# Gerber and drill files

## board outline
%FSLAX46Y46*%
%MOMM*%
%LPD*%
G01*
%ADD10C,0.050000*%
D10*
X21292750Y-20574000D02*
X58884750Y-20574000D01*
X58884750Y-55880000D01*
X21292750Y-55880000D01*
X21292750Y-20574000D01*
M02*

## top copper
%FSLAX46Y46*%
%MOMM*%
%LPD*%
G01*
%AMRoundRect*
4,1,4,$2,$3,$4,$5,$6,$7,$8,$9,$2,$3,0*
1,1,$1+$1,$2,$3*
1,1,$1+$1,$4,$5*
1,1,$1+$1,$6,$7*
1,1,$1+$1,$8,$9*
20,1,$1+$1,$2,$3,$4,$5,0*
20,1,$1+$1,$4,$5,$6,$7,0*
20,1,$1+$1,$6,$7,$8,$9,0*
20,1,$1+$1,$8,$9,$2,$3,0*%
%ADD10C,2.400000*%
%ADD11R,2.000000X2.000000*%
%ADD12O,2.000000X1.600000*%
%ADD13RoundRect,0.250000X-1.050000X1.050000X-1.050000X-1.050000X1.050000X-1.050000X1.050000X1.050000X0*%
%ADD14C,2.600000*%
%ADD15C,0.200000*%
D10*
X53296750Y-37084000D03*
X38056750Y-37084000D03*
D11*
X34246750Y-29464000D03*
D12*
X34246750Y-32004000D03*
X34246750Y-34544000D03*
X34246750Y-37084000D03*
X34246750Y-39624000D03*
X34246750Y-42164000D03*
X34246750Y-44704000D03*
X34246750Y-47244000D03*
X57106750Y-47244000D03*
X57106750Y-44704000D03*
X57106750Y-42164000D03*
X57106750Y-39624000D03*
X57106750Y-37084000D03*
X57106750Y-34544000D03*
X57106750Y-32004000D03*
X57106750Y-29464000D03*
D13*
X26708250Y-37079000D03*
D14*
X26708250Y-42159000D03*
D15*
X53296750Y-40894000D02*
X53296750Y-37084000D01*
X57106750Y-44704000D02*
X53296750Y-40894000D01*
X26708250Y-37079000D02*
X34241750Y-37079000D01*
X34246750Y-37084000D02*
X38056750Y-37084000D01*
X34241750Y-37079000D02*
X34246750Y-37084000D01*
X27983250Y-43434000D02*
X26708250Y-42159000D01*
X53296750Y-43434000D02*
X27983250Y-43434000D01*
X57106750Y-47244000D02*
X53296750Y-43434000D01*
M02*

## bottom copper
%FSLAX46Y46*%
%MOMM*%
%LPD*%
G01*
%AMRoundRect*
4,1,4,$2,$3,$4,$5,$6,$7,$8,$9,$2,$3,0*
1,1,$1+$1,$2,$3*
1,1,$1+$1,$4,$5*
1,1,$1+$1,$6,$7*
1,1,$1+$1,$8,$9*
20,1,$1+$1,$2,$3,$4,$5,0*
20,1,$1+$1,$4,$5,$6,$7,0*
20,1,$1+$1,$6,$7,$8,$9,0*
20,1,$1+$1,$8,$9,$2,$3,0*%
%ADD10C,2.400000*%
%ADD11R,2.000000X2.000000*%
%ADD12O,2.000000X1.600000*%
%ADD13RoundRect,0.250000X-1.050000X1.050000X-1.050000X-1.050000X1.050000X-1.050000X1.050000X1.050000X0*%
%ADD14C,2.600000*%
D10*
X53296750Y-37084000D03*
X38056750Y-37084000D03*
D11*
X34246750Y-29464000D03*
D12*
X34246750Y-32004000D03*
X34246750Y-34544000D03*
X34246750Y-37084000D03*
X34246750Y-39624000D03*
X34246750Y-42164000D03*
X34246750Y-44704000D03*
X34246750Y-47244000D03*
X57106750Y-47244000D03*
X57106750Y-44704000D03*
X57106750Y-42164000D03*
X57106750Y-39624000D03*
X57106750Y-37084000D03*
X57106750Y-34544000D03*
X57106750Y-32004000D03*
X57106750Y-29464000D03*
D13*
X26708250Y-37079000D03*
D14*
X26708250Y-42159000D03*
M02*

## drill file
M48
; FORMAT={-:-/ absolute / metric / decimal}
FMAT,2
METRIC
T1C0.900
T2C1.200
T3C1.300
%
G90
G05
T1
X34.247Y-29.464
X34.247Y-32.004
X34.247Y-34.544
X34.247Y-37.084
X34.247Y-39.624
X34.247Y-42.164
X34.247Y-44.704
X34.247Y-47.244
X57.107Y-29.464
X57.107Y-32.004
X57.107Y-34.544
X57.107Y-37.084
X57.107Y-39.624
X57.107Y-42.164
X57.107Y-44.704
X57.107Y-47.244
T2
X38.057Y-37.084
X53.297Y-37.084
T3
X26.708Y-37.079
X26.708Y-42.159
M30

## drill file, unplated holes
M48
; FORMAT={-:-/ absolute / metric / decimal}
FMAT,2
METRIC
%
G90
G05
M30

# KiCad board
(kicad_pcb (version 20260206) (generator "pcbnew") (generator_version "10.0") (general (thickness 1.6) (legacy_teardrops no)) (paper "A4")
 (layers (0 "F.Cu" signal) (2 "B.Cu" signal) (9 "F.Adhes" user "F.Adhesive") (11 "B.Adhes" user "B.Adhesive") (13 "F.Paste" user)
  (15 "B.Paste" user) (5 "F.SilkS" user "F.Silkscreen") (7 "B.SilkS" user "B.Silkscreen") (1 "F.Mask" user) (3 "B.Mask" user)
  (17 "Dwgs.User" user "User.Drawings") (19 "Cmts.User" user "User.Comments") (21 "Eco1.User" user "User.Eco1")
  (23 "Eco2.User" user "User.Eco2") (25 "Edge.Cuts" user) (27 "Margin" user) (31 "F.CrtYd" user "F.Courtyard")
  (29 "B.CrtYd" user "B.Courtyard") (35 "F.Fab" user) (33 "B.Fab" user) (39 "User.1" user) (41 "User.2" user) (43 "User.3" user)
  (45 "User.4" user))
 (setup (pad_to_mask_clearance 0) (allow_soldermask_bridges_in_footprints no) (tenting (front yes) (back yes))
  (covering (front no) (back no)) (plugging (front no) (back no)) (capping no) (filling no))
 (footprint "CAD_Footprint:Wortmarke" (layer "F.Cu") (at 26.924 49.022)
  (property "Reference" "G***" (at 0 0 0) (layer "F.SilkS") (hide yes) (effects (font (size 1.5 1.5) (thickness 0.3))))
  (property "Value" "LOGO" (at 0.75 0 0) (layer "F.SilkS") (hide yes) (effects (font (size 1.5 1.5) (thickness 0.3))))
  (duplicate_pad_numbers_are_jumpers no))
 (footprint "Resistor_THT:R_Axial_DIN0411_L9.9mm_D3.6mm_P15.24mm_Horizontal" (layer "F.Cu") (at 53.29675 37.084 180)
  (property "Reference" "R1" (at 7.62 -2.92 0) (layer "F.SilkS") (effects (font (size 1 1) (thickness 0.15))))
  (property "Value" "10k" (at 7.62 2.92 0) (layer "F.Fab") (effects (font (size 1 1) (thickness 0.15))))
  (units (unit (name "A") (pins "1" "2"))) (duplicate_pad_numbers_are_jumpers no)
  (pad "1" thru_hole circle (at 0 0 180) (size 2.4 2.4) (drill 1.2) (layers "*.Cu" "*.Mask") (remove_unused_layers no) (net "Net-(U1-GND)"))
  (pad "2" thru_hole circle (at 15.24 0 180) (size 2.4 2.4) (drill 1.2) (layers "*.Cu" "*.Mask") (remove_unused_layers no)
   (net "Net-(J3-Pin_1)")))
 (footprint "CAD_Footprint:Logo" (layer "F.Cu") (at 26.924 27.432)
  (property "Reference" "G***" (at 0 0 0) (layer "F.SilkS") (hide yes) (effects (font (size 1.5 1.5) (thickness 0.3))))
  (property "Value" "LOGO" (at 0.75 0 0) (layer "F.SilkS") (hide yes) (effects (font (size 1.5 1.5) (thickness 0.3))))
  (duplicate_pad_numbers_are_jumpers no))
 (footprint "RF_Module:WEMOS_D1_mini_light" (layer "F.Cu") (at 34.24675 29.464)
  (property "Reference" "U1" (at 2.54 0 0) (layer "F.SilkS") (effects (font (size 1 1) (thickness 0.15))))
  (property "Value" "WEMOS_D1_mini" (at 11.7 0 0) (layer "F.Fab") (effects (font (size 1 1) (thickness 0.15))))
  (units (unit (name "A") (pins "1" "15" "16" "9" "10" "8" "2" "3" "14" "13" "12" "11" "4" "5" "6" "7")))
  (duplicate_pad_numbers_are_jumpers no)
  (pad "1" thru_hole rect (at 0 0) (size 2 2) (drill 0.9) (layers "*.Cu" "*.Mask") (remove_unused_layers no)
   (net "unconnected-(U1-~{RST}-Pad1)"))
  (pad "2" thru_hole oval (at 0 2.54) (size 2 1.6) (drill 0.9) (layers "*.Cu" "*.Mask") (remove_unused_layers no)
   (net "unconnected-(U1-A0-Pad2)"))
  (pad "3" thru_hole oval (at 0 5.08) (size 2 1.6) (drill 0.9) (layers "*.Cu" "*.Mask") (remove_unused_layers no)
   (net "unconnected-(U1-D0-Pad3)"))
  (pad "4" thru_hole oval (at 0 7.62) (size 2 1.6) (drill 0.9) (layers "*.Cu" "*.Mask") (remove_unused_layers no) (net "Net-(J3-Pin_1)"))
  (pad "5" thru_hole oval (at 0 10.16) (size 2 1.6) (drill 0.9) (layers "*.Cu" "*.Mask") (remove_unused_layers no)
   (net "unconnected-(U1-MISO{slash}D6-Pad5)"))
  (pad "6" thru_hole oval (at 0 12.7) (size 2 1.6) (drill 0.9) (layers "*.Cu" "*.Mask") (remove_unused_layers no)
   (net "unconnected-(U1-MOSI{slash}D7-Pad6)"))
  (pad "7" thru_hole oval (at 0 15.24) (size 2 1.6) (drill 0.9) (layers "*.Cu" "*.Mask") (remove_unused_layers no)
   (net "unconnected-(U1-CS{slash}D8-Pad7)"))
  (pad "8" thru_hole oval (at 0 17.78) (size 2 1.6) (drill 0.9) (layers "*.Cu" "*.Mask") (remove_unused_layers no)
   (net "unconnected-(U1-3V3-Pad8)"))
  (pad "9" thru_hole oval (at 22.86 17.78) (size 2 1.6) (drill 0.9) (layers "*.Cu" "*.Mask") (remove_unused_layers no)
   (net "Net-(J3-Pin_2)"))
  (pad "10" thru_hole oval (at 22.86 15.24) (size 2 1.6) (drill 0.9) (layers "*.Cu" "*.Mask") (remove_unused_layers no) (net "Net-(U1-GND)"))
  (pad "11" thru_hole oval (at 22.86 12.7) (size 2 1.6) (drill 0.9) (layers "*.Cu" "*.Mask") (remove_unused_layers no)
   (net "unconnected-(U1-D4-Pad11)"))
  (pad "12" thru_hole oval (at 22.86 10.16) (size 2 1.6) (drill 0.9) (layers "*.Cu" "*.Mask") (remove_unused_layers no)
   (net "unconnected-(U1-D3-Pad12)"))
  (pad "13" thru_hole oval (at 22.86 7.62) (size 2 1.6) (drill 0.9) (layers "*.Cu" "*.Mask") (remove_unused_layers no)
   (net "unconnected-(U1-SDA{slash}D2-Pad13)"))
  (pad "14" thru_hole oval (at 22.86 5.08) (size 2 1.6) (drill 0.9) (layers "*.Cu" "*.Mask") (remove_unused_layers no)
   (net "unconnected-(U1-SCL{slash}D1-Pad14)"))
  (pad "15" thru_hole oval (at 22.86 2.54) (size 2 1.6) (drill 0.9) (layers "*.Cu" "*.Mask") (remove_unused_layers no)
   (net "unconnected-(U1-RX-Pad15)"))
  (pad "16" thru_hole oval (at 22.86 0) (size 2 1.6) (drill 0.9) (layers "*.Cu" "*.Mask") (remove_unused_layers no)
   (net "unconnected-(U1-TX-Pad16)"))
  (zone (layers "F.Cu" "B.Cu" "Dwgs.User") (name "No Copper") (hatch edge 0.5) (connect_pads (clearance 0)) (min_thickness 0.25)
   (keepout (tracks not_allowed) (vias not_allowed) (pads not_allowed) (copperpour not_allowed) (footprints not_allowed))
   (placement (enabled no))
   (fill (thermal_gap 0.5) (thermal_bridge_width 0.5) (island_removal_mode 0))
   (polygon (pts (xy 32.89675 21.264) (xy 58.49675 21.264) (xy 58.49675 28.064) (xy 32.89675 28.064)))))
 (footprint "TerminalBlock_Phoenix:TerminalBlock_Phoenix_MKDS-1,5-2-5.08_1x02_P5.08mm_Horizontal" (layer "F.Cu") (at 26.70825 37.079 -90)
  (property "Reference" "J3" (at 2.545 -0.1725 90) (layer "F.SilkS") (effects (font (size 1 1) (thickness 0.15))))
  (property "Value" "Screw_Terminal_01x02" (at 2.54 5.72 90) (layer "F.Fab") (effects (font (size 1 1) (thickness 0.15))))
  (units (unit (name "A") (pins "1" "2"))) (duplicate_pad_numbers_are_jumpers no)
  (pad "1" thru_hole roundrect (at 0 0 270) (size 2.6 2.6) (drill 1.3) (layers "*.Cu" "*.Mask") (remove_unused_layers no)
   (roundrect_rratio 0.096154) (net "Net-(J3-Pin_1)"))
  (pad "2" thru_hole circle (at 5.08 0 270) (size 2.6 2.6) (drill 1.3) (layers "*.Cu" "*.Mask") (remove_unused_layers no)
   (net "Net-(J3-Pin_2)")))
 (gr_rect (start 21.29275 20.574) (end 58.88475 55.88) (stroke (width 0.05) (type default)) (fill no) (layer "Edge.Cuts"))
 (segment (start 53.29675 40.894) (end 53.29675 37.084) (width 0.2) (layer "F.Cu") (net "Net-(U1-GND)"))
 (segment (start 57.10675 44.704) (end 53.29675 40.894) (width 0.2) (layer "F.Cu") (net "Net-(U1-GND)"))
 (segment (start 26.70825 37.079) (end 34.24175 37.079) (width 0.2) (layer "F.Cu") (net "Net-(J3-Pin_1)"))
 (segment (start 34.24675 37.084) (end 38.05675 37.084) (width 0.2) (layer "F.Cu") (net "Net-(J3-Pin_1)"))
 (segment (start 34.24175 37.079) (end 34.24675 37.084) (width 0.2) (layer "F.Cu") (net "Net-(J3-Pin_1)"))
 (segment (start 27.98325 43.434) (end 26.70825 42.159) (width 0.2) (layer "F.Cu") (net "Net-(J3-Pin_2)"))
 (segment (start 53.29675 43.434) (end 27.98325 43.434) (width 0.2) (layer "F.Cu") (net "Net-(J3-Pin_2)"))
 (segment (start 57.10675 47.244) (end 53.29675 43.434) (width 0.2) (layer "F.Cu") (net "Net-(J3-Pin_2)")))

